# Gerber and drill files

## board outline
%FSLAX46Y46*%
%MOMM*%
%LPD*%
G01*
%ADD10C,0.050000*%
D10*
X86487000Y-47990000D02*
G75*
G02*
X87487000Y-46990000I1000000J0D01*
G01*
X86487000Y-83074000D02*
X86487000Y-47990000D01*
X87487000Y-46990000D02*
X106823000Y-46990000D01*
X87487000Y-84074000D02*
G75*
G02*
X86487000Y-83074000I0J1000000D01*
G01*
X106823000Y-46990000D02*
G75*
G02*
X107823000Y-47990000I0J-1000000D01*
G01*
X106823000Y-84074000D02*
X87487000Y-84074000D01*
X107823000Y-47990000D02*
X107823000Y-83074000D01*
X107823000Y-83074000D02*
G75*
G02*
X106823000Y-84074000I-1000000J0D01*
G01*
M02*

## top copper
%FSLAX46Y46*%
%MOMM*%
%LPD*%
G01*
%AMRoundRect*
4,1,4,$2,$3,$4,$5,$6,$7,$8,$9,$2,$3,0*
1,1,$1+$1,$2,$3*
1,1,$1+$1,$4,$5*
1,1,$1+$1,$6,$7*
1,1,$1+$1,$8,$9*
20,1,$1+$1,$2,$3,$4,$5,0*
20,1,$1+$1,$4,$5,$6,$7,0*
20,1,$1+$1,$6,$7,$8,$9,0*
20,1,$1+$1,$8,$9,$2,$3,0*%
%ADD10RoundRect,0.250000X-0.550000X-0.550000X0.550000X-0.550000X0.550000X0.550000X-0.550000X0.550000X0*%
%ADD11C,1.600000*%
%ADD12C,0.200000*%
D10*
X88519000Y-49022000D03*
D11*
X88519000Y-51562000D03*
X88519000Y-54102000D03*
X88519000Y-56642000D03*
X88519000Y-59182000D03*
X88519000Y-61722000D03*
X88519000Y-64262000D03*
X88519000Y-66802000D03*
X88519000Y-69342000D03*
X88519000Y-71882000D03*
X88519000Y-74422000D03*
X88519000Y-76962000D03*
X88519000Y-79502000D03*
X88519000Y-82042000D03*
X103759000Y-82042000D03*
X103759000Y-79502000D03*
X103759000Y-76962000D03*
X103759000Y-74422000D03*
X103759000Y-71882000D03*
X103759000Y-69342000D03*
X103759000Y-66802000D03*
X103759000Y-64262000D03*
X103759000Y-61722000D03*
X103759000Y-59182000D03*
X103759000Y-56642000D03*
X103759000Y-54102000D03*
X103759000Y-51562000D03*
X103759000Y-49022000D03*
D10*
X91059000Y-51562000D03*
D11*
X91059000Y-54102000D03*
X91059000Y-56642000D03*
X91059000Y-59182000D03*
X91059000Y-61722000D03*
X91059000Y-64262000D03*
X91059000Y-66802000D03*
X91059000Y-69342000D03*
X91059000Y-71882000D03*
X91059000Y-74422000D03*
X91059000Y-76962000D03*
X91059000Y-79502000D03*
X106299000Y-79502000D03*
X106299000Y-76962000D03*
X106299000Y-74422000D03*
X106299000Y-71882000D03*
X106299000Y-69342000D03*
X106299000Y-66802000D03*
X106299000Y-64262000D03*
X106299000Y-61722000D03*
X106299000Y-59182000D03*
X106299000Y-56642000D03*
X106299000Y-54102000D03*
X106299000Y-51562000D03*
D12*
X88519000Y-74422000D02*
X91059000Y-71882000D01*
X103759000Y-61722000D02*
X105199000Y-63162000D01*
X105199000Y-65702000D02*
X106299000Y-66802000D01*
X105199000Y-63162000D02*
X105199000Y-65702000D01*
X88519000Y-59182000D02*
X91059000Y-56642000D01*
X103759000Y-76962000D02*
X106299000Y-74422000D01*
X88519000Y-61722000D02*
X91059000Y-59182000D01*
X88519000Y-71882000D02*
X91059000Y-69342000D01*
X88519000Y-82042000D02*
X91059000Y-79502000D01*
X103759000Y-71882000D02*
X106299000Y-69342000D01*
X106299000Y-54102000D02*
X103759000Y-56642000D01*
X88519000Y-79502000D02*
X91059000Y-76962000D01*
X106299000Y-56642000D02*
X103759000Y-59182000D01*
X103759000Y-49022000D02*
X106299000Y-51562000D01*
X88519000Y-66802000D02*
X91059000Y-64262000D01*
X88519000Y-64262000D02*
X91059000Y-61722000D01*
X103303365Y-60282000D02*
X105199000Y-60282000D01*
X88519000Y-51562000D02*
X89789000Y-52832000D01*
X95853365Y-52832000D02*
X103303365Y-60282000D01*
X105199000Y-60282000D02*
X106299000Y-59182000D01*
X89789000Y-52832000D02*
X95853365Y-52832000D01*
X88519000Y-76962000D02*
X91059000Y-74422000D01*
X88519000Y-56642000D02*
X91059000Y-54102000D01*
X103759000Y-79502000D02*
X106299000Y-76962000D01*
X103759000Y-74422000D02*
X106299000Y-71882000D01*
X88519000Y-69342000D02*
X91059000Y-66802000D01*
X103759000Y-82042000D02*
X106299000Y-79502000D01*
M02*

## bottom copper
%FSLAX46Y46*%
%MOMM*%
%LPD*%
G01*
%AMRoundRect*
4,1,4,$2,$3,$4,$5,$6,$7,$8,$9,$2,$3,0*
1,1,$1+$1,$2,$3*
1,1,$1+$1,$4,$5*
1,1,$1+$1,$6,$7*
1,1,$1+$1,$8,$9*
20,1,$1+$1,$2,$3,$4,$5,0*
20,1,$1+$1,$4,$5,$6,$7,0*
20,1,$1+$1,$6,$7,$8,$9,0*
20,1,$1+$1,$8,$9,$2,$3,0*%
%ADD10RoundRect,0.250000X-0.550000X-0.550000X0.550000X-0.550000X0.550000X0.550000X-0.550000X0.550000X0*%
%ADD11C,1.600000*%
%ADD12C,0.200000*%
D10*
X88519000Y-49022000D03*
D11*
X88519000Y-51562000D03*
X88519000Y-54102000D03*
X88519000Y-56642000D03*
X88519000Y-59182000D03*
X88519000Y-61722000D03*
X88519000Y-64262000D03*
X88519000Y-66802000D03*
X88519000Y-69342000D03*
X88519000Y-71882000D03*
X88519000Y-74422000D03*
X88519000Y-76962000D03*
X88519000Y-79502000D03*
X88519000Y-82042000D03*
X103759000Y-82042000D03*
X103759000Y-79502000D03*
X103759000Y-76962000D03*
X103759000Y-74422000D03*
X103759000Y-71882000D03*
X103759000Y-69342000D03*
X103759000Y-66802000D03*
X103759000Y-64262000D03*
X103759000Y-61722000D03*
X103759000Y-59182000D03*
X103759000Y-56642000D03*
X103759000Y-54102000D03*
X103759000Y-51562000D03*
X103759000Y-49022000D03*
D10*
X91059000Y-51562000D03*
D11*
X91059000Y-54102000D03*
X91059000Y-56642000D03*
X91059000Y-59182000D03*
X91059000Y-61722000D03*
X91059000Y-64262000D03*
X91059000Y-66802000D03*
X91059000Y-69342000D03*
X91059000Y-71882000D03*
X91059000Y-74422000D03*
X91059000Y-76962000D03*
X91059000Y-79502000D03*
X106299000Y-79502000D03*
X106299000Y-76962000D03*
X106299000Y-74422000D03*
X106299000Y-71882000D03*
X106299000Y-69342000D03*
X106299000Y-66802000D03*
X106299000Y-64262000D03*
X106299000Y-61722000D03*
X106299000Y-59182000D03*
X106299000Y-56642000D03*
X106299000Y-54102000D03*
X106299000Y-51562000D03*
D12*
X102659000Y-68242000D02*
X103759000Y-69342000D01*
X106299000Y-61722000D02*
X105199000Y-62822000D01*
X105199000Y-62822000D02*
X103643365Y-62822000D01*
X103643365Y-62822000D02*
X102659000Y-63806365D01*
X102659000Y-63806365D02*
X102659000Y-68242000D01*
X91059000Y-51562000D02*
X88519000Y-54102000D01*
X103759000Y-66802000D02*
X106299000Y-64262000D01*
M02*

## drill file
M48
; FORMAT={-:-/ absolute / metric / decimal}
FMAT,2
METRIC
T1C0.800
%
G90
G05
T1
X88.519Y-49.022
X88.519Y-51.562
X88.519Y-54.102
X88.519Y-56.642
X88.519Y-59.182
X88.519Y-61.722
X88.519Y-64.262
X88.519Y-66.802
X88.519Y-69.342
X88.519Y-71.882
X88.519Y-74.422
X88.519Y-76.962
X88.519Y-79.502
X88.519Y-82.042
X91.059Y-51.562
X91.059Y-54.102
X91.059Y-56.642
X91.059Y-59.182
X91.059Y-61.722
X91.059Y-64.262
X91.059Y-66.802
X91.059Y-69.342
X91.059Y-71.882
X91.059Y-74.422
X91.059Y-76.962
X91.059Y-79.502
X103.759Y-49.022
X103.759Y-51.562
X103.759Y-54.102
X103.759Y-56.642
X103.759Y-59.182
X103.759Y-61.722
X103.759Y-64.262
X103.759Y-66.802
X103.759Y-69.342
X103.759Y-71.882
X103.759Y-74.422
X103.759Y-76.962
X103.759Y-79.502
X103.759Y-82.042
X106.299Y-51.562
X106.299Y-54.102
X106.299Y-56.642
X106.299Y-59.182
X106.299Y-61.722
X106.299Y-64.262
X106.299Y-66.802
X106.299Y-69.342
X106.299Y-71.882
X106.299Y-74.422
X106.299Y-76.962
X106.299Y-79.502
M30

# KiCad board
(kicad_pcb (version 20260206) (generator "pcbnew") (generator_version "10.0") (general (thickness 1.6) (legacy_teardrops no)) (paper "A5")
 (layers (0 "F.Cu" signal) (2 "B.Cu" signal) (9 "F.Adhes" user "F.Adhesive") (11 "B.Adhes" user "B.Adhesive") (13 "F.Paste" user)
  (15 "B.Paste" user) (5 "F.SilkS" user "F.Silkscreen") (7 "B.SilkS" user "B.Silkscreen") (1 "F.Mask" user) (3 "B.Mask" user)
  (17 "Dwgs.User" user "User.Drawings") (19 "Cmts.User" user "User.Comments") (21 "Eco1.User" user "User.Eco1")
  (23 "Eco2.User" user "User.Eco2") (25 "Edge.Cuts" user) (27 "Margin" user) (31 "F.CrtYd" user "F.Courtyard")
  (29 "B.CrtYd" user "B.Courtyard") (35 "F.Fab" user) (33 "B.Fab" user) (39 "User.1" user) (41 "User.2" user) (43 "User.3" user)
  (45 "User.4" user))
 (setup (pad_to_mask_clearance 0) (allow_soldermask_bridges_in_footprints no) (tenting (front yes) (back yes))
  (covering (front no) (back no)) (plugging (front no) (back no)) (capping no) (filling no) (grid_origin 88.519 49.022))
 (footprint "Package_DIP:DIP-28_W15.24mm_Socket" (layer "F.Cu") (at 88.519 49.022)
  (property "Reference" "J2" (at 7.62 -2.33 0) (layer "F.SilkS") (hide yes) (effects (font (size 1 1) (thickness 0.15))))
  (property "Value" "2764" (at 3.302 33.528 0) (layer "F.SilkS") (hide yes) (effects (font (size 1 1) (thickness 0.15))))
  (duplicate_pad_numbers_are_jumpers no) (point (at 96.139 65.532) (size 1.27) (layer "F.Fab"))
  (pad "1" thru_hole roundrect (at 0 0) (size 1.6 1.6) (drill 0.8) (layers "*.Cu" "*.Mask") (remove_unused_layers no)
   (roundrect_rratio 0.15625) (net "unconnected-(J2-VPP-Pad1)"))
  (pad "2" thru_hole circle (at 0 2.54) (size 1.6 1.6) (drill 0.8) (layers "*.Cu" "*.Mask") (remove_unused_layers no) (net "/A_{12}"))
  (pad "3" thru_hole circle (at 0 5.08) (size 1.6 1.6) (drill 0.8) (layers "*.Cu" "*.Mask") (remove_unused_layers no) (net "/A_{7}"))
  (pad "4" thru_hole circle (at 0 7.62) (size 1.6 1.6) (drill 0.8) (layers "*.Cu" "*.Mask") (remove_unused_layers no) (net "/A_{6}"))
  (pad "5" thru_hole circle (at 0 10.16) (size 1.6 1.6) (drill 0.8) (layers "*.Cu" "*.Mask") (remove_unused_layers no) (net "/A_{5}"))
  (pad "6" thru_hole circle (at 0 12.7) (size 1.6 1.6) (drill 0.8) (layers "*.Cu" "*.Mask") (remove_unused_layers no) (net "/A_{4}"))
  (pad "7" thru_hole circle (at 0 15.24) (size 1.6 1.6) (drill 0.8) (layers "*.Cu" "*.Mask") (remove_unused_layers no) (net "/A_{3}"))
  (pad "8" thru_hole circle (at 0 17.78) (size 1.6 1.6) (drill 0.8) (layers "*.Cu" "*.Mask") (remove_unused_layers no) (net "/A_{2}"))
  (pad "9" thru_hole circle (at 0 20.32) (size 1.6 1.6) (drill 0.8) (layers "*.Cu" "*.Mask") (remove_unused_layers no) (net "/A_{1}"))
  (pad "10" thru_hole circle (at 0 22.86) (size 1.6 1.6) (drill 0.8) (layers "*.Cu" "*.Mask") (remove_unused_layers no) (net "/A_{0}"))
  (pad "11" thru_hole circle (at 0 25.4) (size 1.6 1.6) (drill 0.8) (layers "*.Cu" "*.Mask") (remove_unused_layers no) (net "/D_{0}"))
  (pad "12" thru_hole circle (at 0 27.94) (size 1.6 1.6) (drill 0.8) (layers "*.Cu" "*.Mask") (remove_unused_layers no) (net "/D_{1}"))
  (pad "13" thru_hole circle (at 0 30.48) (size 1.6 1.6) (drill 0.8) (layers "*.Cu" "*.Mask") (remove_unused_layers no) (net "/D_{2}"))
  (pad "14" thru_hole circle (at 0 33.02) (size 1.6 1.6) (drill 0.8) (layers "*.Cu" "*.Mask") (remove_unused_layers no) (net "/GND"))
  (pad "15" thru_hole circle (at 15.24 33.02) (size 1.6 1.6) (drill 0.8) (layers "*.Cu" "*.Mask") (remove_unused_layers no) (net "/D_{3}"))
  (pad "16" thru_hole circle (at 15.24 30.48) (size 1.6 1.6) (drill 0.8) (layers "*.Cu" "*.Mask") (remove_unused_layers no) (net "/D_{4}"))
  (pad "17" thru_hole circle (at 15.24 27.94) (size 1.6 1.6) (drill 0.8) (layers "*.Cu" "*.Mask") (remove_unused_layers no) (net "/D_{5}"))
  (pad "18" thru_hole circle (at 15.24 25.4) (size 1.6 1.6) (drill 0.8) (layers "*.Cu" "*.Mask") (remove_unused_layers no) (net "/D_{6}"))
  (pad "19" thru_hole circle (at 15.24 22.86) (size 1.6 1.6) (drill 0.8) (layers "*.Cu" "*.Mask") (remove_unused_layers no) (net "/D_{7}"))
  (pad "20" thru_hole circle (at 15.24 20.32) (size 1.6 1.6) (drill 0.8) (layers "*.Cu" "*.Mask") (remove_unused_layers no) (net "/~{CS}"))
  (pad "21" thru_hole circle (at 15.24 17.78) (size 1.6 1.6) (drill 0.8) (layers "*.Cu" "*.Mask") (remove_unused_layers no) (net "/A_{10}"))
  (pad "22" thru_hole circle (at 15.24 15.24) (size 1.6 1.6) (drill 0.8) (layers "*.Cu" "*.Mask") (remove_unused_layers no)
   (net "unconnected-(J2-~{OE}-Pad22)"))
  (pad "23" thru_hole circle (at 15.24 12.7) (size 1.6 1.6) (drill 0.8) (layers "*.Cu" "*.Mask") (remove_unused_layers no) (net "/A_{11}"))
  (pad "24" thru_hole circle (at 15.24 10.16) (size 1.6 1.6) (drill 0.8) (layers "*.Cu" "*.Mask") (remove_unused_layers no) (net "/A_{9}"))
  (pad "25" thru_hole circle (at 15.24 7.62) (size 1.6 1.6) (drill 0.8) (layers "*.Cu" "*.Mask") (remove_unused_layers no) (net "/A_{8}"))
  (pad "26" thru_hole circle (at 15.24 5.08) (size 1.6 1.6) (drill 0.8) (layers "*.Cu" "*.Mask") (remove_unused_layers no)
   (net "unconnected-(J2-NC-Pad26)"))
  (pad "27" thru_hole circle (at 15.24 2.54) (size 1.6 1.6) (drill 0.8) (layers "*.Cu" "*.Mask") (remove_unused_layers no)
   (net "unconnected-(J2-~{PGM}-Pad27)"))
  (pad "28" thru_hole circle (at 15.24 0) (size 1.6 1.6) (drill 0.8) (layers "*.Cu" "*.Mask") (remove_unused_layers no) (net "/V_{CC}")))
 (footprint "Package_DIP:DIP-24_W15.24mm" (layer "F.Cu") (at 91.059 51.562)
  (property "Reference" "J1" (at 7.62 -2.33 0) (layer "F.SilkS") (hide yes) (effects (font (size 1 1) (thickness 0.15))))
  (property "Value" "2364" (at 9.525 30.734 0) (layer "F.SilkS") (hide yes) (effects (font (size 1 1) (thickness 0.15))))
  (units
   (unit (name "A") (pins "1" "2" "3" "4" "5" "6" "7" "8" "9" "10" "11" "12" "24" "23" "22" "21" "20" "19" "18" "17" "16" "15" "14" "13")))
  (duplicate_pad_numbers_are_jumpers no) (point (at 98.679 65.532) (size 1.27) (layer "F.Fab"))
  (pad "1" thru_hole roundrect (at 0 0) (size 1.6 1.6) (drill 0.8) (layers "*.Cu" "*.Mask") (remove_unused_layers no)
   (roundrect_rratio 0.15625) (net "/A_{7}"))
  (pad "2" thru_hole circle (at 0 2.54) (size 1.6 1.6) (drill 0.8) (layers "*.Cu" "*.Mask") (remove_unused_layers no) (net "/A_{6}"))
  (pad "3" thru_hole circle (at 0 5.08) (size 1.6 1.6) (drill 0.8) (layers "*.Cu" "*.Mask") (remove_unused_layers no) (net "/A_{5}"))
  (pad "4" thru_hole circle (at 0 7.62) (size 1.6 1.6) (drill 0.8) (layers "*.Cu" "*.Mask") (remove_unused_layers no) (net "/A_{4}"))
  (pad "5" thru_hole circle (at 0 10.16) (size 1.6 1.6) (drill 0.8) (layers "*.Cu" "*.Mask") (remove_unused_layers no) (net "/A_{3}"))
  (pad "6" thru_hole circle (at 0 12.7) (size 1.6 1.6) (drill 0.8) (layers "*.Cu" "*.Mask") (remove_unused_layers no) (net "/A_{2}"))
  (pad "7" thru_hole circle (at 0 15.24) (size 1.6 1.6) (drill 0.8) (layers "*.Cu" "*.Mask") (remove_unused_layers no) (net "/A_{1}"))
  (pad "8" thru_hole circle (at 0 17.78) (size 1.6 1.6) (drill 0.8) (layers "*.Cu" "*.Mask") (remove_unused_layers no) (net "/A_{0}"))
  (pad "9" thru_hole circle (at 0 20.32) (size 1.6 1.6) (drill 0.8) (layers "*.Cu" "*.Mask") (remove_unused_layers no) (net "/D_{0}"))
  (pad "10" thru_hole circle (at 0 22.86) (size 1.6 1.6) (drill 0.8) (layers "*.Cu" "*.Mask") (remove_unused_layers no) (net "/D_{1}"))
  (pad "11" thru_hole circle (at 0 25.4) (size 1.6 1.6) (drill 0.8) (layers "*.Cu" "*.Mask") (remove_unused_layers no) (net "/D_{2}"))
  (pad "12" thru_hole circle (at 0 27.94) (size 1.6 1.6) (drill 0.8) (layers "*.Cu" "*.Mask") (remove_unused_layers no) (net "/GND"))
  (pad "13" thru_hole circle (at 15.24 27.94) (size 1.6 1.6) (drill 0.8) (layers "*.Cu" "*.Mask") (remove_unused_layers no) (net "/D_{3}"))
  (pad "14" thru_hole circle (at 15.24 25.4) (size 1.6 1.6) (drill 0.8) (layers "*.Cu" "*.Mask") (remove_unused_layers no) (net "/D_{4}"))
  (pad "15" thru_hole circle (at 15.24 22.86) (size 1.6 1.6) (drill 0.8) (layers "*.Cu" "*.Mask") (remove_unused_layers no) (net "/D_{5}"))
  (pad "16" thru_hole circle (at 15.24 20.32) (size 1.6 1.6) (drill 0.8) (layers "*.Cu" "*.Mask") (remove_unused_layers no) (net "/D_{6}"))
  (pad "17" thru_hole circle (at 15.24 17.78) (size 1.6 1.6) (drill 0.8) (layers "*.Cu" "*.Mask") (remove_unused_layers no) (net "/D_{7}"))
  (pad "18" thru_hole circle (at 15.24 15.24) (size 1.6 1.6) (drill 0.8) (layers "*.Cu" "*.Mask") (remove_unused_layers no) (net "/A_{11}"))
  (pad "19" thru_hole circle (at 15.24 12.7) (size 1.6 1.6) (drill 0.8) (layers "*.Cu" "*.Mask") (remove_unused_layers no) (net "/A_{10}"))
  (pad "20" thru_hole circle (at 15.24 10.16) (size 1.6 1.6) (drill 0.8) (layers "*.Cu" "*.Mask") (remove_unused_layers no) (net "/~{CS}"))
  (pad "21" thru_hole circle (at 15.24 7.62) (size 1.6 1.6) (drill 0.8) (layers "*.Cu" "*.Mask") (remove_unused_layers no) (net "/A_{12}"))
  (pad "22" thru_hole circle (at 15.24 5.08) (size 1.6 1.6) (drill 0.8) (layers "*.Cu" "*.Mask") (remove_unused_layers no) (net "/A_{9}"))
  (pad "23" thru_hole circle (at 15.24 2.54) (size 1.6 1.6) (drill 0.8) (layers "*.Cu" "*.Mask") (remove_unused_layers no) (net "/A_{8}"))
  (pad "24" thru_hole circle (at 15.24 0) (size 1.6 1.6) (drill 0.8) (layers "*.Cu" "*.Mask") (remove_unused_layers no) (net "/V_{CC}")))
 (gr_arc (start 86.487 47.99) (mid 86.779893 47.282893) (end 87.487 46.99) (stroke (width 0.05) (type default)) (layer "Edge.Cuts"))
 (gr_line (start 86.487 83.074) (end 86.487 47.99) (stroke (width 0.05) (type default)) (layer "Edge.Cuts"))
 (gr_line (start 87.487 46.99) (end 106.823 46.99) (stroke (width 0.05) (type default)) (layer "Edge.Cuts"))
 (gr_arc (start 87.487 84.074) (mid 86.779893 83.781107) (end 86.487 83.074) (stroke (width 0.05) (type default)) (layer "Edge.Cuts"))
 (gr_arc (start 106.823 46.99) (mid 107.530107 47.282893) (end 107.823 47.99) (stroke (width 0.05) (type default)) (layer "Edge.Cuts"))
 (gr_line (start 106.823 84.074) (end 87.487 84.074) (stroke (width 0.05) (type default)) (layer "Edge.Cuts"))
 (gr_line (start 107.823 47.99) (end 107.823 83.074) (stroke (width 0.05) (type default)) (layer "Edge.Cuts"))
 (gr_arc (start 107.823 83.074) (mid 107.530107 83.781107) (end 106.823 84.074) (stroke (width 0.05) (type default)) (layer "Edge.Cuts"))
 (segment (start 88.519 74.422) (end 91.059 71.882) (width 0.2) (layer "F.Cu") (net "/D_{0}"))
 (segment (start 103.759 61.722) (end 105.199 63.162) (width 0.2) (layer "F.Cu") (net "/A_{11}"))
 (segment (start 105.199 65.702) (end 106.299 66.802) (width 0.2) (layer "F.Cu") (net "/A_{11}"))
 (segment (start 105.199 63.162) (end 105.199 65.702) (width 0.2) (layer "F.Cu") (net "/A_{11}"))
 (segment (start 88.519 59.182) (end 91.059 56.642) (width 0.2) (layer "F.Cu") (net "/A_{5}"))
 (segment (start 103.759 76.962) (end 106.299 74.422) (width 0.2) (layer "F.Cu") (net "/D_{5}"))
 (segment (start 88.519 61.722) (end 91.059 59.182) (width 0.2) (layer "F.Cu") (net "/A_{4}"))
 (segment (start 88.519 71.882) (end 91.059 69.342) (width 0.2) (layer "F.Cu") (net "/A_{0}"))
 (segment (start 88.519 82.042) (end 91.059 79.502) (width 0.2) (layer "F.Cu") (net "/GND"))
 (segment (start 103.759 71.882) (end 106.299 69.342) (width 0.2) (layer "F.Cu") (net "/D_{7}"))
 (segment (start 102.659 68.242) (end 103.759 69.342) (width 0.2) (layer "B.Cu") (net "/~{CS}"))
 (segment (start 106.299 61.722) (end 105.199 62.822) (width 0.2) (layer "B.Cu") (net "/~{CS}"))
 (segment (start 105.199 62.822) (end 103.643365 62.822) (width 0.2) (layer "B.Cu") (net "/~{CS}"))
 (segment (start 103.643365 62.822) (end 102.659 63.806365) (width 0.2) (layer "B.Cu") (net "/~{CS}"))
 (segment (start 102.659 63.806365) (end 102.659 68.242) (width 0.2) (layer "B.Cu") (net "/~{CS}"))
 (segment (start 91.059 51.562) (end 88.519 54.102) (width 0.2) (layer "B.Cu") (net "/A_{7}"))
 (segment (start 106.299 54.102) (end 103.759 56.642) (width 0.2) (layer "F.Cu") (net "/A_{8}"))
 (segment (start 88.519 79.502) (end 91.059 76.962) (width 0.2) (layer "F.Cu") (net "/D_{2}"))
 (segment (start 106.299 56.642) (end 103.759 59.182) (width 0.2) (layer "F.Cu") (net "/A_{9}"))
 (segment (start 103.759 49.022) (end 106.299 51.562) (width 0.2) (layer "F.Cu") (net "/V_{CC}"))
 (segment (start 103.759 66.802) (end 106.299 64.262) (width 0.2) (layer "B.Cu") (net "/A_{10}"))
 (segment (start 88.519 66.802) (end 91.059 64.262) (width 0.2) (layer "F.Cu") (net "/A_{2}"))
 (segment (start 88.519 64.262) (end 91.059 61.722) (width 0.2) (layer "F.Cu") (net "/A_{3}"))
 (segment (start 103.303365 60.282) (end 105.199 60.282) (width 0.2) (layer "F.Cu") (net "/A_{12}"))
 (segment (start 88.519 51.562) (end 89.789 52.832) (width 0.2) (layer "F.Cu") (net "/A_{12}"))
 (segment (start 95.853365 52.832) (end 103.303365 60.282) (width 0.2) (layer "F.Cu") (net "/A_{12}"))
 (segment (start 105.199 60.282) (end 106.299 59.182) (width 0.2) (layer "F.Cu") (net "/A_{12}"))
 (segment (start 89.789 52.832) (end 95.853365 52.832) (width 0.2) (layer "F.Cu") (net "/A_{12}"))
 (segment (start 88.519 76.962) (end 91.059 74.422) (width 0.2) (layer "F.Cu") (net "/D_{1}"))
 (segment (start 88.519 56.642) (end 91.059 54.102) (width 0.2) (layer "F.Cu") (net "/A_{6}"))
 (segment (start 103.759 79.502) (end 106.299 76.962) (width 0.2) (layer "F.Cu") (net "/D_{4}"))
 (segment (start 103.759 74.422) (end 106.299 71.882) (width 0.2) (layer "F.Cu") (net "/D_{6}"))
 (segment (start 88.519 69.342) (end 91.059 66.802) (width 0.2) (layer "F.Cu") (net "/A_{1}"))
 (segment (start 103.759 82.042) (end 106.299 79.502) (width 0.2) (layer "F.Cu") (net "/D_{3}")))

